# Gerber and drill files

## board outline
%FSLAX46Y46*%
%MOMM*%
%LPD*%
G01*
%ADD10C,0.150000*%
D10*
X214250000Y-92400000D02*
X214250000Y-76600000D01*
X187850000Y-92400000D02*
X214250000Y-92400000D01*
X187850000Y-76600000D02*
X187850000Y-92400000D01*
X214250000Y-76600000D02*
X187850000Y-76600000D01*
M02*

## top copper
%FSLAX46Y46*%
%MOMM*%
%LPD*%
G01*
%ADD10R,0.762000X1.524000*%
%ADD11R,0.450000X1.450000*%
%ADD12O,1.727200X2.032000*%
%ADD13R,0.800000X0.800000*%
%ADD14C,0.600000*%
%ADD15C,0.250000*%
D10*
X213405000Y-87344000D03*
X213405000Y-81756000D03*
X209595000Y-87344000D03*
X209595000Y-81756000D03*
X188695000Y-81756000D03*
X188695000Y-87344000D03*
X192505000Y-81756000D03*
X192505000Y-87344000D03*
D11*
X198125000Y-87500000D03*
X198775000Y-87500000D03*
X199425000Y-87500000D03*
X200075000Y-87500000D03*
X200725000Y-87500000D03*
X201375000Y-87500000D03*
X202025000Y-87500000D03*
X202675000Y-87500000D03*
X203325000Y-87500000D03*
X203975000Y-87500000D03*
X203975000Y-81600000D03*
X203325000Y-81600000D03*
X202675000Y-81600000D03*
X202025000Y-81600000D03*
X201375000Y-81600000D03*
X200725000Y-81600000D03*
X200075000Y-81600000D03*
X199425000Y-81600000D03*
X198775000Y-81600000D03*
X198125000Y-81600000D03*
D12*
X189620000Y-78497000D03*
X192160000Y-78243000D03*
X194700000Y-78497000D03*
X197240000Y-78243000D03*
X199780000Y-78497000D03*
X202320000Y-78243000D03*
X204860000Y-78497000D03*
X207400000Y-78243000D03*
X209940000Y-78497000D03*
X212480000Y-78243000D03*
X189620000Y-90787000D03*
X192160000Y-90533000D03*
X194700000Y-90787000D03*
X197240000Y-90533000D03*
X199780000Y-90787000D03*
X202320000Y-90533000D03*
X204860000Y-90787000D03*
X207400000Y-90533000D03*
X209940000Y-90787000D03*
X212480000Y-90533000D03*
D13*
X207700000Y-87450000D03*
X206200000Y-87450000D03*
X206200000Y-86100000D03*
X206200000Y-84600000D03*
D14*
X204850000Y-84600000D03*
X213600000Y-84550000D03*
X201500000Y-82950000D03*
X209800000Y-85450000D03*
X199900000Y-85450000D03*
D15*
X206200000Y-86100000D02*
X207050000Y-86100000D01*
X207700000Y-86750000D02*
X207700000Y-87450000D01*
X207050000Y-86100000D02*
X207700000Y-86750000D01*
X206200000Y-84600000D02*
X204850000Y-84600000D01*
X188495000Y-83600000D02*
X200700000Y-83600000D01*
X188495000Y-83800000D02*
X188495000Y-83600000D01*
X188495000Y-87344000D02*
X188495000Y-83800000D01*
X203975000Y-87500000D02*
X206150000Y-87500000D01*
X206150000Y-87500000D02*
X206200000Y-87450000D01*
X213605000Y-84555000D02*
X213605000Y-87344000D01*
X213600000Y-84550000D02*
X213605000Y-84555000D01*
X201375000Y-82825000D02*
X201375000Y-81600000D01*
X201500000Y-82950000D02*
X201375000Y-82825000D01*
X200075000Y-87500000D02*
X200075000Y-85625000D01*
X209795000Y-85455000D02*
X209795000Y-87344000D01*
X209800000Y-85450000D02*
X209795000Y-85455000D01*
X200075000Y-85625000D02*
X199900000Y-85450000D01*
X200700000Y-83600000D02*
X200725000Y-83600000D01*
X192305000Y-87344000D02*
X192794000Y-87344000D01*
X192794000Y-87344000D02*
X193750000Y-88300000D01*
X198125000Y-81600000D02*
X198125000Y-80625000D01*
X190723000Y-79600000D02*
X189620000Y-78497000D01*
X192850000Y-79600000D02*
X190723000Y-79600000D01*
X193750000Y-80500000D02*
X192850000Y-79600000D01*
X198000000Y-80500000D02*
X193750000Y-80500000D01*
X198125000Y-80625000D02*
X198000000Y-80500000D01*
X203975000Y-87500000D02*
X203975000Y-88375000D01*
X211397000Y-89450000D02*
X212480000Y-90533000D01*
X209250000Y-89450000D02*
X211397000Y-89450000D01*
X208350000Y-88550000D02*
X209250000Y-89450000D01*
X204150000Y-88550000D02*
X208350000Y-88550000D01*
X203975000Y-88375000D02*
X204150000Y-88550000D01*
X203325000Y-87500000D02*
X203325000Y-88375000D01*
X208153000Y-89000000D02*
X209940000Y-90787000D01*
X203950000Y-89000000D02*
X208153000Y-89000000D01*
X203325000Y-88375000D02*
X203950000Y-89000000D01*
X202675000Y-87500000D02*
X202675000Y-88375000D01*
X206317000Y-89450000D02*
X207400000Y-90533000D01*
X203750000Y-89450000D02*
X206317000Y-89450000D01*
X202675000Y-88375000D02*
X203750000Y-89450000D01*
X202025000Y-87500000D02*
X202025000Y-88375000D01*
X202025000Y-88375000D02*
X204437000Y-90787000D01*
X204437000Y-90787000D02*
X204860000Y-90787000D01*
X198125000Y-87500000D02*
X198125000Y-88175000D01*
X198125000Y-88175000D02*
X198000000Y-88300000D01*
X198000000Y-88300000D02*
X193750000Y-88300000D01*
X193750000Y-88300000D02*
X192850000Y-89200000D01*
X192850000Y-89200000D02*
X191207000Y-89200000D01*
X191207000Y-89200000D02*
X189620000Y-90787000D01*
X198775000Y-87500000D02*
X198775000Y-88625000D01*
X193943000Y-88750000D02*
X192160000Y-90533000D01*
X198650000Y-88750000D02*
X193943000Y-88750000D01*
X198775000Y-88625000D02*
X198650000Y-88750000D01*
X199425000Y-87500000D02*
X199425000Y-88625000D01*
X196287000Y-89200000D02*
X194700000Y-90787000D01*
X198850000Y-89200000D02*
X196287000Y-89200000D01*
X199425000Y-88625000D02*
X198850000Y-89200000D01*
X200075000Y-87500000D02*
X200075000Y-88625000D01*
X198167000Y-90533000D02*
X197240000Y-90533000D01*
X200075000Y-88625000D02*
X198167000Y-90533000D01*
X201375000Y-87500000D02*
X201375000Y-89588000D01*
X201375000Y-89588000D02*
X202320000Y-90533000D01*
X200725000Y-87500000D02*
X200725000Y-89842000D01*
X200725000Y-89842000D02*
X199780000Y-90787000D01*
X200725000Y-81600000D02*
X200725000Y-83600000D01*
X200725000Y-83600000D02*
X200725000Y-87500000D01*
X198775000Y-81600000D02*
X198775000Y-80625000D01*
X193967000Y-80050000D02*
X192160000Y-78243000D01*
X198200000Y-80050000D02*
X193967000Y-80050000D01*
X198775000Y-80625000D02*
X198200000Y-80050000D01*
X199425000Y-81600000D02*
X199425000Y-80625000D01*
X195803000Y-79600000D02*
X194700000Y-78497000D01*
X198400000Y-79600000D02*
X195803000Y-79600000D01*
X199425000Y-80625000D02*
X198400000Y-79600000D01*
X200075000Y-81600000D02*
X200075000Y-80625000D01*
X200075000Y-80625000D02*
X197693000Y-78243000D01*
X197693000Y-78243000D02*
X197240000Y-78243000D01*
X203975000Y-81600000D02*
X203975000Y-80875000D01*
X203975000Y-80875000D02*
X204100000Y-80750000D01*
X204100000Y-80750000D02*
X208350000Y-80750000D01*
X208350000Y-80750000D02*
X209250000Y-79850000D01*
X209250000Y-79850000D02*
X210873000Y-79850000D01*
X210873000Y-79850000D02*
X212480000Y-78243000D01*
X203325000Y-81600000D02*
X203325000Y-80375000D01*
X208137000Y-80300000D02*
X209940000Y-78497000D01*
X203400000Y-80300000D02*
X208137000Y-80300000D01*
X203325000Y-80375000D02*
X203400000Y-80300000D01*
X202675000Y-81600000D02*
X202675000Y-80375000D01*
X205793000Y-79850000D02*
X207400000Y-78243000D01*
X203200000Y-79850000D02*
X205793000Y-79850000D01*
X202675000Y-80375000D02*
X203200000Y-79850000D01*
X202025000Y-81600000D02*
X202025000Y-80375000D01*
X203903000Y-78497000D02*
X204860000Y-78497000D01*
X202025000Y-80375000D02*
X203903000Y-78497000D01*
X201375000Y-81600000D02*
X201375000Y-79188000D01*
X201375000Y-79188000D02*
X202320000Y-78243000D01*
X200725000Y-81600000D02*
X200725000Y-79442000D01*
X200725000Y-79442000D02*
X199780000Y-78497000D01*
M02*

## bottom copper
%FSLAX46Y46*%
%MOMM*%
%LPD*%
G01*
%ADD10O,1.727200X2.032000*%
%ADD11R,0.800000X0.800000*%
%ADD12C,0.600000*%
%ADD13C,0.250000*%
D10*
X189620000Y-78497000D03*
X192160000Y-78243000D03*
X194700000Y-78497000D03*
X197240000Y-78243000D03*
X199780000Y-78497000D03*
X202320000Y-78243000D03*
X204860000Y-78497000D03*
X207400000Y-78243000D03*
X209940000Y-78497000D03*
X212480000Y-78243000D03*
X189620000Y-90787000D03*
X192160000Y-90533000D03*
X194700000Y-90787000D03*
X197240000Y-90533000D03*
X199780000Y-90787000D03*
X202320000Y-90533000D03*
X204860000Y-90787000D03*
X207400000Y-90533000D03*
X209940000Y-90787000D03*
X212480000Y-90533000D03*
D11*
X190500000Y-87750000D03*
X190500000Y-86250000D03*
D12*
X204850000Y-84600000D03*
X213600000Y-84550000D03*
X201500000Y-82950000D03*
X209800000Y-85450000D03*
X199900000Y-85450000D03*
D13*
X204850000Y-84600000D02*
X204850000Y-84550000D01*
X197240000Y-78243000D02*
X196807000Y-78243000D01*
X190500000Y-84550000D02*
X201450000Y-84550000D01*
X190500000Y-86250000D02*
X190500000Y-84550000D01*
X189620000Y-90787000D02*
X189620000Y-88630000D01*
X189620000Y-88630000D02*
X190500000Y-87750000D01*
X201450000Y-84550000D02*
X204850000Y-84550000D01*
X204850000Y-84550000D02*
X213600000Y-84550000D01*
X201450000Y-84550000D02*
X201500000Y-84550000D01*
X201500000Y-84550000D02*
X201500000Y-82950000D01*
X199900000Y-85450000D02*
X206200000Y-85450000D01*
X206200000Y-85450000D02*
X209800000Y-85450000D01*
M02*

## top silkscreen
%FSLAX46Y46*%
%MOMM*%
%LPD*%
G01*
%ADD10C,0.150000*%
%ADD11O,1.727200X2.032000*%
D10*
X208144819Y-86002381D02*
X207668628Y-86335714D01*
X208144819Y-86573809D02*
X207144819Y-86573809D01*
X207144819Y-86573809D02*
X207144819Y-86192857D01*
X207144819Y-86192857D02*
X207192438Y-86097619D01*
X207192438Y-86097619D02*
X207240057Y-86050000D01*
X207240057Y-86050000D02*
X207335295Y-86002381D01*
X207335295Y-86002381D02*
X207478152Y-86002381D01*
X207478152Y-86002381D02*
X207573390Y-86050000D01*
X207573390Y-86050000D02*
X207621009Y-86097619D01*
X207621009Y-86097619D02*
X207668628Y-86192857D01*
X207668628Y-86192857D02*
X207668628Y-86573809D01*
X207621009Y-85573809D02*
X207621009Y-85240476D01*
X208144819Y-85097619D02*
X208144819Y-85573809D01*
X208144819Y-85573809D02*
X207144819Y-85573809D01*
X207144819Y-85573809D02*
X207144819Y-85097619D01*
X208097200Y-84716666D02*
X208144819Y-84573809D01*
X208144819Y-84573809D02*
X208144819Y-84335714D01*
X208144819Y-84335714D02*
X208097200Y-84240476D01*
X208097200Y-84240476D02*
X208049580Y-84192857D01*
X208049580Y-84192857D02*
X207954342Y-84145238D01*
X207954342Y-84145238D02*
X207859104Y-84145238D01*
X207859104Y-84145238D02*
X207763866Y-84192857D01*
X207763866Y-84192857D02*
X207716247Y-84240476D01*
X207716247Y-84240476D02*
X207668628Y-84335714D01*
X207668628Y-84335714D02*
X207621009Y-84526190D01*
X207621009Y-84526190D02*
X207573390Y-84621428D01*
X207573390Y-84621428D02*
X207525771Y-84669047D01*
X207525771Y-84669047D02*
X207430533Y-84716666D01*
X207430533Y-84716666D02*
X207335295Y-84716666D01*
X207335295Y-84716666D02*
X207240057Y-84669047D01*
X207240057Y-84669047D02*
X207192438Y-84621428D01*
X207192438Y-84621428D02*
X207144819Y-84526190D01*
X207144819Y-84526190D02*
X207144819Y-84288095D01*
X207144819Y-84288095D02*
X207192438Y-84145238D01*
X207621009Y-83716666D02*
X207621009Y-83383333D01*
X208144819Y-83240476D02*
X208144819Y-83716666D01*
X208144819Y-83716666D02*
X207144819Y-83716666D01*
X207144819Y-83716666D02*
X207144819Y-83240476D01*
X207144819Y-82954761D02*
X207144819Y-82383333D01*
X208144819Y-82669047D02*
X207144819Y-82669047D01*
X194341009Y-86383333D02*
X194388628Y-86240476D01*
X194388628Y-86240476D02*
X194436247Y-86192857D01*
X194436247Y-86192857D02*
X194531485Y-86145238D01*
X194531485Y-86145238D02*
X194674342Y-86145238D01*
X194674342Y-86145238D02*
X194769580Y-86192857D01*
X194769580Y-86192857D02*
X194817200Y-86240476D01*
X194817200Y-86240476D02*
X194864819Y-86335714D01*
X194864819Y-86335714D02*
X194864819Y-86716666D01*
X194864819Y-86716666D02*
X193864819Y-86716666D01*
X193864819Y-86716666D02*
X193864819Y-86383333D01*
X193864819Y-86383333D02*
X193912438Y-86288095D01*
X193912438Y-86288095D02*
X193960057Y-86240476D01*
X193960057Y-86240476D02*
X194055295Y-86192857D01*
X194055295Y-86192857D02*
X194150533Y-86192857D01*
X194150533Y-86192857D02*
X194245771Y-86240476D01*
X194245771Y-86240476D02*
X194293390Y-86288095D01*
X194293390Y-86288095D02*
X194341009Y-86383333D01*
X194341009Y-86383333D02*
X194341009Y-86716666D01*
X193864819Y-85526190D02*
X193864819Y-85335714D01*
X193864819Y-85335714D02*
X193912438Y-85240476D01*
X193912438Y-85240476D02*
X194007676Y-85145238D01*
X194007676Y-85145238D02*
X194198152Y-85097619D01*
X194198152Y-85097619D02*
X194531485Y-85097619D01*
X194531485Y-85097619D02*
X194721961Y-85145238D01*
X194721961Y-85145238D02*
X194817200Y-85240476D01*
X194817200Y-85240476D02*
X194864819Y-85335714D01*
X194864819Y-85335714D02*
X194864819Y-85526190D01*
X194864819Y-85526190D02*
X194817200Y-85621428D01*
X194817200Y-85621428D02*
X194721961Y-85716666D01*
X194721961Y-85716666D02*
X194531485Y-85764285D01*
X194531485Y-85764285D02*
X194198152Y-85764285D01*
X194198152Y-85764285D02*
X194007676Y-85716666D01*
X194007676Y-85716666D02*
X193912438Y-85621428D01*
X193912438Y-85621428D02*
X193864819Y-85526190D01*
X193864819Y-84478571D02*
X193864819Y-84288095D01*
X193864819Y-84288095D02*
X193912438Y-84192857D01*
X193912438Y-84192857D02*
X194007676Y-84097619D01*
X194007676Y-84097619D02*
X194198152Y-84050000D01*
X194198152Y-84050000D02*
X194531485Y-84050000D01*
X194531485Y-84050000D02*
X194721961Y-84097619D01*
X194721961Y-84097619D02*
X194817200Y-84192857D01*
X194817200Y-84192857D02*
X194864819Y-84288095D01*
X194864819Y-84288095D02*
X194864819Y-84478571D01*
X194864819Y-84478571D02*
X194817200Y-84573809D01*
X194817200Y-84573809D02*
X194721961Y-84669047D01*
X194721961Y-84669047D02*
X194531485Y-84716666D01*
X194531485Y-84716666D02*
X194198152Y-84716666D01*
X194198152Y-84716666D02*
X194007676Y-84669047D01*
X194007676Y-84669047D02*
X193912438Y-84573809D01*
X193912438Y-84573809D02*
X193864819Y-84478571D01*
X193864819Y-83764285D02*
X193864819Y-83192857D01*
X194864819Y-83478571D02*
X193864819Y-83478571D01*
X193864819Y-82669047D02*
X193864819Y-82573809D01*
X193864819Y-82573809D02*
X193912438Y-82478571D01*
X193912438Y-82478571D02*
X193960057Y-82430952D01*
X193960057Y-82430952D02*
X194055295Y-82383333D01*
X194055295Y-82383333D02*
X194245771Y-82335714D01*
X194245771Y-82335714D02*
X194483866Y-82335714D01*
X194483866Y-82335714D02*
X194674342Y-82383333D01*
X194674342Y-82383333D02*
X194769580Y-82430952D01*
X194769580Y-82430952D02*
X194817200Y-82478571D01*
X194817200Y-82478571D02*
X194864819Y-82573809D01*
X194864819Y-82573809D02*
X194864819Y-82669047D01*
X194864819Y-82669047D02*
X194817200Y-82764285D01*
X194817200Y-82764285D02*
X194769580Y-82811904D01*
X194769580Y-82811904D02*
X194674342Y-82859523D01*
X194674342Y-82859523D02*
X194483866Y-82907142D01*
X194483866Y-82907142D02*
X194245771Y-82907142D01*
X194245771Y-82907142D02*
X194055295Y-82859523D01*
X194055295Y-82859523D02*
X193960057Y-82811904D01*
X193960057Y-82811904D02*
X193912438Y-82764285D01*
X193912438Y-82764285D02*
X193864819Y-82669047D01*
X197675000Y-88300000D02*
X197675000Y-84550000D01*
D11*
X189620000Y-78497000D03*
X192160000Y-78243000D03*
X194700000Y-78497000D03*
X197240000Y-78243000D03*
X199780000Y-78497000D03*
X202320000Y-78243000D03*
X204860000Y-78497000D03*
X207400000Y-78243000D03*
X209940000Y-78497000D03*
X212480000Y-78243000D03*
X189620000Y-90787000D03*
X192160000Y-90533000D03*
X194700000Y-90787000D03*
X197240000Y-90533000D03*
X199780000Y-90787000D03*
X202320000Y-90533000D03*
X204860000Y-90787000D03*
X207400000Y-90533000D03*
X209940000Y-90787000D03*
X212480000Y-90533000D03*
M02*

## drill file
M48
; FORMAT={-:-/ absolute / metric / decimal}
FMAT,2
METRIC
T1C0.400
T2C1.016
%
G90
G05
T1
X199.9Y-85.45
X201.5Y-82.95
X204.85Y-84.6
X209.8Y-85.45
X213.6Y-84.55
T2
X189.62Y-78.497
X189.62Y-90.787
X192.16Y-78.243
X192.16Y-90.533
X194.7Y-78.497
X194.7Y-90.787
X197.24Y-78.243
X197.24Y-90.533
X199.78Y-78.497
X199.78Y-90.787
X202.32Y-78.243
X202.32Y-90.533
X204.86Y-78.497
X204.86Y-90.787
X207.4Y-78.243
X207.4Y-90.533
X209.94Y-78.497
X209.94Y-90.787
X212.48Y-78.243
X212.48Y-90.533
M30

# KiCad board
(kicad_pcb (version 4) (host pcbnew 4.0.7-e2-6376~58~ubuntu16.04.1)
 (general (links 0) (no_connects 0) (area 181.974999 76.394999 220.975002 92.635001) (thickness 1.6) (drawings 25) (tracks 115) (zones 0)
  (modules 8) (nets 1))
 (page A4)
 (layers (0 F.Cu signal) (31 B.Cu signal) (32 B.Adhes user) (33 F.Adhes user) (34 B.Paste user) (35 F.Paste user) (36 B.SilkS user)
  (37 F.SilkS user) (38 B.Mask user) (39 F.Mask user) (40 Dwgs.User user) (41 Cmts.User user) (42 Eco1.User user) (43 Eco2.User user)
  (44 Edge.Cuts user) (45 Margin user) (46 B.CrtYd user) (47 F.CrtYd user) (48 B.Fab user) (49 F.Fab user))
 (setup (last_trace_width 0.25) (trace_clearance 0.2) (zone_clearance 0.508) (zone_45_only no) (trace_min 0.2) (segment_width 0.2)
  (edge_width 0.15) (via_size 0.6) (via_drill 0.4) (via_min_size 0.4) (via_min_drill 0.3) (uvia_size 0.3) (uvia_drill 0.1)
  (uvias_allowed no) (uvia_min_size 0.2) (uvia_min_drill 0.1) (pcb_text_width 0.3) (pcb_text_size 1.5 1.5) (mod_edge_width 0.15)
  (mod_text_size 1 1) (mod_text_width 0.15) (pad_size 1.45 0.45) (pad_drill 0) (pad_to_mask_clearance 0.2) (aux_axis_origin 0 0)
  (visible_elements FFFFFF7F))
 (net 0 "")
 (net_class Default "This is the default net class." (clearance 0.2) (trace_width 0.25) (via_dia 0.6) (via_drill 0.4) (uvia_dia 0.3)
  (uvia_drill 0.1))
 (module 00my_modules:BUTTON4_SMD (layer F.Cu) (at 211.5 84.55 90)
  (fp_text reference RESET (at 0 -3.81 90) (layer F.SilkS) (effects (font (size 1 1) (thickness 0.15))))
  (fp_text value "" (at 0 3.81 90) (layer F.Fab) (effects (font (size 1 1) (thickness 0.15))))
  (pad 1 smd rect (at -2.794 1.905 90) (size 1.524 0.762) (layers F.Cu F.Paste F.Mask))
  (pad 2 smd rect (at 2.794 1.905 90) (size 1.524 0.762) (layers F.Cu F.Paste F.Mask))
  (pad 3 smd rect (at -2.794 -1.905 90) (size 1.524 0.762) (layers F.Cu F.Paste F.Mask))
  (pad 4 smd rect (at 2.794 -1.905 90) (size 1.524 0.762) (layers F.Cu F.Paste F.Mask)))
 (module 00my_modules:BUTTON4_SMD (layer F.Cu) (at 190.6 84.55 270)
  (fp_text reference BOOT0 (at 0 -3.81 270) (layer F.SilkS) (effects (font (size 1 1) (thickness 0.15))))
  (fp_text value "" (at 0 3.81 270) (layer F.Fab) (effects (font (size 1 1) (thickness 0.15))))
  (pad 1 smd rect (at -2.794 1.905 270) (size 1.524 0.762) (layers F.Cu F.Paste F.Mask))
  (pad 2 smd rect (at 2.794 1.905 270) (size 1.524 0.762) (layers F.Cu F.Paste F.Mask))
  (pad 3 smd rect (at -2.794 -1.905 270) (size 1.524 0.762) (layers F.Cu F.Paste F.Mask))
  (pad 4 smd rect (at 2.794 -1.905 270) (size 1.524 0.762) (layers F.Cu F.Paste F.Mask)))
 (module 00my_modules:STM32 (layer F.Cu) (at 201.05 84.55 90)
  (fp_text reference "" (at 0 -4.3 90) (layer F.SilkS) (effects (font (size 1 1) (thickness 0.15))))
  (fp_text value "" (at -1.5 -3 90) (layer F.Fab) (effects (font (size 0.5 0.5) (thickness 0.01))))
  (fp_line (start -3.75 -3.375) (end 0 -3.375) (layer F.SilkS) (width 0.15))
  (pad BOOT smd rect (at -2.95 -2.925 90) (size 1.45 0.45) (layers F.Cu F.Paste F.Mask))
  (pad PF0 smd rect (at -2.95 -2.275 90) (size 1.45 0.45) (layers F.Cu F.Paste F.Mask))
  (pad PF1 smd rect (at -2.95 -1.625 90) (size 1.45 0.45) (layers F.Cu F.Paste F.Mask))
  (pad NRST smd rect (at -2.95 -0.975 90) (size 1.45 0.45) (layers F.Cu F.Paste F.Mask))
  (pad VCC smd rect (at -2.95 -0.325 90) (size 1.45 0.45) (layers F.Cu F.Paste F.Mask))
  (pad PA0 smd rect (at -2.95 0.325 90) (size 1.45 0.45) (layers F.Cu F.Paste F.Mask))
  (pad PA1 smd rect (at -2.95 0.975 90) (size 1.45 0.45) (layers F.Cu F.Paste F.Mask))
  (pad PA2 smd rect (at -2.95 1.625 90) (size 1.45 0.45) (layers F.Cu F.Paste F.Mask))
  (pad PA3 smd rect (at -2.95 2.275 90) (size 1.45 0.45) (layers F.Cu F.Paste F.Mask))
  (pad PA4 smd rect (at -2.95 2.925 90) (size 1.45 0.45) (layers F.Cu F.Paste F.Mask))
  (pad PA5 smd rect (at 2.95 2.925 90) (size 1.45 0.45) (layers F.Cu F.Paste F.Mask))
  (pad PA6 smd rect (at 2.95 2.275 90) (size 1.45 0.45) (layers F.Cu F.Paste F.Mask))
  (pad PA7 smd rect (at 2.95 1.625 90) (size 1.45 0.45) (layers F.Cu F.Paste F.Mask))
  (pad PB1 smd rect (at 2.95 0.975 90) (size 1.45 0.45) (layers F.Cu F.Paste F.Mask))
  (pad GND smd rect (at 2.95 0.325 90) (size 1.45 0.45) (layers F.Cu F.Paste F.Mask))
  (pad VCC smd rect (at 2.95 -0.325 90) (size 1.45 0.45) (layers F.Cu F.Paste F.Mask))
  (pad TX smd rect (at 2.95 -0.975 90) (size 1.45 0.45) (layers F.Cu F.Paste F.Mask))
  (pad RX smd rect (at 2.95 -1.625 90) (size 1.45 0.45) (layers F.Cu F.Paste F.Mask))
  (pad DIO smd rect (at 2.95 -2.275 90) (size 1.45 0.45) (layers F.Cu F.Paste F.Mask))
  (pad CLK smd rect (at 2.95 -2.925 90) (size 1.45 0.45) (layers F.Cu F.Paste F.Mask)))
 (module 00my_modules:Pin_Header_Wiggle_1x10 (layer F.Cu) (at 189.62 78.37 90)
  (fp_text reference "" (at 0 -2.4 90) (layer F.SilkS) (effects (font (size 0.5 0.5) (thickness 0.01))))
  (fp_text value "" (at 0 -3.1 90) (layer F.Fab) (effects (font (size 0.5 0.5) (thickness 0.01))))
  (pad 1 thru_hole oval (at -0.127 0 90) (size 2.032 1.7272) (drill 1.016) (layers *.Cu *.Mask F.SilkS))
  (pad 2 thru_hole oval (at 0.127 2.54 90) (size 2.032 1.7272) (drill 1.016) (layers *.Cu *.Mask F.SilkS))
  (pad 3 thru_hole oval (at -0.127 5.08 90) (size 2.032 1.7272) (drill 1.016) (layers *.Cu *.Mask F.SilkS))
  (pad 4 thru_hole oval (at 0.127 7.62 90) (size 2.032 1.7272) (drill 1.016) (layers *.Cu *.Mask F.SilkS))
  (pad 5 thru_hole oval (at -0.127 10.16 90) (size 2.032 1.7272) (drill 1.016) (layers *.Cu *.Mask F.SilkS))
  (pad 6 thru_hole oval (at 0.127 12.7 90) (size 2.032 1.7272) (drill 1.016) (layers *.Cu *.Mask F.SilkS))
  (pad 7 thru_hole oval (at -0.127 15.24 90) (size 2.032 1.7272) (drill 1.016) (layers *.Cu *.Mask F.SilkS))
  (pad 8 thru_hole oval (at 0.127 17.78 90) (size 2.032 1.7272) (drill 1.016) (layers *.Cu *.Mask F.SilkS))
  (pad 9 thru_hole oval (at -0.127 20.32 90) (size 2.032 1.7272) (drill 1.016) (layers *.Cu *.Mask F.SilkS))
  (pad 10 thru_hole oval (at 0.127 22.86 90) (size 2.032 1.7272) (drill 1.016) (layers *.Cu *.Mask F.SilkS)))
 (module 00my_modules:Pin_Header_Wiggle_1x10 (layer F.Cu) (at 189.62 90.66 90)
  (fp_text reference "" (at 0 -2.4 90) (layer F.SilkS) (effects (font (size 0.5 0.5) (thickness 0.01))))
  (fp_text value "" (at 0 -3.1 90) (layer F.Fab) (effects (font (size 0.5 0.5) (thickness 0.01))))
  (pad 1 thru_hole oval (at -0.127 0 90) (size 2.032 1.7272) (drill 1.016) (layers *.Cu *.Mask F.SilkS))
  (pad 2 thru_hole oval (at 0.127 2.54 90) (size 2.032 1.7272) (drill 1.016) (layers *.Cu *.Mask F.SilkS))
  (pad 3 thru_hole oval (at -0.127 5.08 90) (size 2.032 1.7272) (drill 1.016) (layers *.Cu *.Mask F.SilkS))
  (pad 4 thru_hole oval (at 0.127 7.62 90) (size 2.032 1.7272) (drill 1.016) (layers *.Cu *.Mask F.SilkS))
  (pad 5 thru_hole oval (at -0.127 10.16 90) (size 2.032 1.7272) (drill 1.016) (layers *.Cu *.Mask F.SilkS))
  (pad 6 thru_hole oval (at 0.127 12.7 90) (size 2.032 1.7272) (drill 1.016) (layers *.Cu *.Mask F.SilkS))
  (pad 7 thru_hole oval (at -0.127 15.24 90) (size 2.032 1.7272) (drill 1.016) (layers *.Cu *.Mask F.SilkS))
  (pad 8 thru_hole oval (at 0.127 17.78 90) (size 2.032 1.7272) (drill 1.016) (layers *.Cu *.Mask F.SilkS))
  (pad 9 thru_hole oval (at -0.127 20.32 90) (size 2.032 1.7272) (drill 1.016) (layers *.Cu *.Mask F.SilkS))
  (pad 10 thru_hole oval (at 0.127 22.86 90) (size 2.032 1.7272) (drill 1.016) (layers *.Cu *.Mask F.SilkS)))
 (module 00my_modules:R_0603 (layer B.Cu) (at 190.5 87 90)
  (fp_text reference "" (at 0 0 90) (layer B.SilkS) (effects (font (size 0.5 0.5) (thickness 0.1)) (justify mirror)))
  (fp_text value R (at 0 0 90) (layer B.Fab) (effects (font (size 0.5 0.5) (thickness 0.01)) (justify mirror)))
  (pad 1 smd rect (at -0.75 0 90) (size 0.8 0.8) (layers B.Cu B.Paste B.Mask))
  (pad 2 smd rect (at 0.75 0 90) (size 0.8 0.8) (layers B.Cu B.Paste B.Mask)))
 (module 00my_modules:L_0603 (layer F.Cu) (at 206.95 87.45 180)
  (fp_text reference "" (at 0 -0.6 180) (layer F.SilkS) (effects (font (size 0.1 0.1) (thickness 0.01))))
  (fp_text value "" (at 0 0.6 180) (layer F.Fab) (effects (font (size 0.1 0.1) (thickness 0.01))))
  (pad 1 smd rect (at -0.75 0 180) (size 0.8 0.8) (layers F.Cu F.Paste F.Mask))
  (pad 2 smd rect (at 0.75 0 180) (size 0.8 0.8) (layers F.Cu F.Paste F.Mask)))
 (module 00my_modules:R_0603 (layer F.Cu) (at 206.2 85.35 90)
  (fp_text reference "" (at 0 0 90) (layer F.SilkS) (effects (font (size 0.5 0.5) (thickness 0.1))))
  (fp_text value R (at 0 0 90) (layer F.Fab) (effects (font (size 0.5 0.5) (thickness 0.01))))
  (pad 1 smd rect (at -0.75 0 90) (size 0.8 0.8) (layers F.Cu F.Paste F.Mask))
  (pad 2 smd rect (at 0.75 0 90) (size 0.8 0.8) (layers F.Cu F.Paste F.Mask)))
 (gr_line (start 214.25 92.4) (end 214.25 76.6) (angle 90) (layer Edge.Cuts) (width 0.15))
 (gr_line (start 187.85 92.4) (end 214.25 92.4) (angle 90) (layer Edge.Cuts) (width 0.15))
 (gr_line (start 187.85 76.6) (end 187.85 92.4) (angle 90) (layer Edge.Cuts) (width 0.15))
 (gr_line (start 214.25 76.6) (end 187.85 76.6) (angle 90) (layer Edge.Cuts) (width 0.15))
 (segment (start 206.2 86.1) (end 207.05 86.1) (width 0.25) (layer F.Cu) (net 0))
 (segment (start 207.7 86.75) (end 207.7 87.45) (width 0.25) (layer F.Cu) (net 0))
 (segment (start 207.05 86.1) (end 207.7 86.75) (width 0.25) (layer F.Cu) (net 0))
 (segment (start 206.2 84.6) (end 204.85 84.6) (width 0.25) (layer F.Cu) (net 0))
 (segment (start 204.85 84.6) (end 204.85 84.55) (width 0.25) (layer B.Cu) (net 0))
 (via (at 204.85 84.6) (size 0.6) (drill 0.4) (layers F.Cu B.Cu) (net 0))
 (segment (start 188.495 83.6) (end 200.7 83.6) (width 0.25) (layer F.Cu) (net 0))
 (segment (start 188.495 83.8) (end 188.495 83.6) (width 0.25) (layer F.Cu) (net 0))
 (segment (start 188.495 87.344) (end 188.495 83.8) (width 0.25) (layer F.Cu) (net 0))
 (segment (start 203.975 87.5) (end 206.15 87.5) (width 0.25) (layer F.Cu) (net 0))
 (segment (start 206.15 87.5) (end 206.2 87.45) (width 0.25) (layer F.Cu) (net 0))
 (segment (start 197.24 78.243) (end 196.807 78.243) (width 0.25) (layer B.Cu) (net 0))
 (segment (start 190.5 84.55) (end 201.45 84.55) (width 0.25) (layer B.Cu) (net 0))
 (segment (start 190.5 86.25) (end 190.5 84.55) (width 0.25) (layer B.Cu) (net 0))
 (segment (start 189.62 90.787) (end 189.62 88.63) (width 0.25) (layer B.Cu) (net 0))
 (segment (start 189.62 88.63) (end 190.5 87.75) (width 0.25) (layer B.Cu) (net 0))
 (segment (start 201.45 84.55) (end 204.85 84.55) (width 0.25) (layer B.Cu) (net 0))
 (segment (start 204.85 84.55) (end 213.6 84.55) (width 0.25) (layer B.Cu) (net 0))
 (via (at 213.6 84.55) (size 0.6) (drill 0.4) (layers F.Cu B.Cu) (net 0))
 (segment (start 213.605 84.555) (end 213.605 87.344) (width 0.25) (layer F.Cu) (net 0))
 (segment (start 213.6 84.55) (end 213.605 84.555) (width 0.25) (layer F.Cu) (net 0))
 (segment (start 201.45 84.55) (end 201.5 84.55) (width 0.25) (layer B.Cu) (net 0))
 (segment (start 201.375 82.825) (end 201.375 81.6) (width 0.25) (layer F.Cu) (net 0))
 (segment (start 201.5 82.95) (end 201.375 82.825) (width 0.25) (layer F.Cu) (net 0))
 (via (at 201.5 82.95) (size 0.6) (drill 0.4) (layers F.Cu B.Cu) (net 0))
 (segment (start 201.5 84.55) (end 201.5 82.95) (width 0.25) (layer B.Cu) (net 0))
 (segment (start 200.075 87.5) (end 200.075 85.625) (width 0.25) (layer F.Cu) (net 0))
 (segment (start 209.795 85.455) (end 209.795 87.344) (width 0.25) (layer F.Cu) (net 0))
 (segment (start 209.8 85.45) (end 209.795 85.455) (width 0.25) (layer F.Cu) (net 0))
 (via (at 209.8 85.45) (size 0.6) (drill 0.4) (layers F.Cu B.Cu) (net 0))
 (segment (start 199.9 85.45) (end 206.2 85.45) (width 0.25) (layer B.Cu) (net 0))
 (segment (start 206.2 85.45) (end 209.8 85.45) (width 0.25) (layer B.Cu) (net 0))
 (via (at 199.9 85.45) (size 0.6) (drill 0.4) (layers F.Cu B.Cu) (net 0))
 (segment (start 200.075 85.625) (end 199.9 85.45) (width 0.25) (layer F.Cu) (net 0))
 (segment (start 200.7 83.6) (end 200.725 83.6) (width 0.25) (layer F.Cu) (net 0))
 (segment (start 192.305 87.344) (end 192.794 87.344) (width 0.25) (layer F.Cu) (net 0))
 (segment (start 192.794 87.344) (end 193.75 88.3) (width 0.25) (layer F.Cu) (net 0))
 (segment (start 198.125 81.6) (end 198.125 80.625) (width 0.25) (layer F.Cu) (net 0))
 (segment (start 190.723 79.6) (end 189.62 78.497) (width 0.25) (layer F.Cu) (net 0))
 (segment (start 192.85 79.6) (end 190.723 79.6) (width 0.25) (layer F.Cu) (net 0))
 (segment (start 193.75 80.5) (end 192.85 79.6) (width 0.25) (layer F.Cu) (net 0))
 (segment (start 198 80.5) (end 193.75 80.5) (width 0.25) (layer F.Cu) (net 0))
 (segment (start 198.125 80.625) (end 198 80.5) (width 0.25) (layer F.Cu) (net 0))
 (segment (start 203.975 87.5) (end 203.975 88.375) (width 0.25) (layer F.Cu) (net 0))
 (segment (start 211.397 89.45) (end 212.48 90.533) (width 0.25) (layer F.Cu) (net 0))
 (segment (start 209.25 89.45) (end 211.397 89.45) (width 0.25) (layer F.Cu) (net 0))
 (segment (start 208.35 88.55) (end 209.25 89.45) (width 0.25) (layer F.Cu) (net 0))
 (segment (start 204.15 88.55) (end 208.35 88.55) (width 0.25) (layer F.Cu) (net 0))
 (segment (start 203.975 88.375) (end 204.15 88.55) (width 0.25) (layer F.Cu) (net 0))
 (segment (start 203.325 87.5) (end 203.325 88.375) (width 0.25) (layer F.Cu) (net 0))
 (segment (start 208.153 89) (end 209.94 90.787) (width 0.25) (layer F.Cu) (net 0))
 (segment (start 203.95 89) (end 208.153 89) (width 0.25) (layer F.Cu) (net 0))
 (segment (start 203.325 88.375) (end 203.95 89) (width 0.25) (layer F.Cu) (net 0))
 (segment (start 202.675 87.5) (end 202.675 88.375) (width 0.25) (layer F.Cu) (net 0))
 (segment (start 206.317 89.45) (end 207.4 90.533) (width 0.25) (layer F.Cu) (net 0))
 (segment (start 203.75 89.45) (end 206.317 89.45) (width 0.25) (layer F.Cu) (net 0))
 (segment (start 202.675 88.375) (end 203.75 89.45) (width 0.25) (layer F.Cu) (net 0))
 (segment (start 202.025 87.5) (end 202.025 88.375) (width 0.25) (layer F.Cu) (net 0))
 (segment (start 202.025 88.375) (end 204.437 90.787) (width 0.25) (layer F.Cu) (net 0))
 (segment (start 204.437 90.787) (end 204.86 90.787) (width 0.25) (layer F.Cu) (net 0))
 (segment (start 198.125 87.5) (end 198.125 88.175) (width 0.25) (layer F.Cu) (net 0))
 (segment (start 198.125 88.175) (end 198 88.3) (width 0.25) (layer F.Cu) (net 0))
 (segment (start 198 88.3) (end 193.75 88.3) (width 0.25) (layer F.Cu) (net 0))
 (segment (start 193.75 88.3) (end 192.85 89.2) (width 0.25) (layer F.Cu) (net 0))
 (segment (start 192.85 89.2) (end 191.207 89.2) (width 0.25) (layer F.Cu) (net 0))
 (segment (start 191.207 89.2) (end 189.62 90.787) (width 0.25) (layer F.Cu) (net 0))
 (segment (start 198.775 87.5) (end 198.775 88.625) (width 0.25) (layer F.Cu) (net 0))
 (segment (start 193.943 88.75) (end 192.16 90.533) (width 0.25) (layer F.Cu) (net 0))
 (segment (start 198.65 88.75) (end 193.943 88.75) (width 0.25) (layer F.Cu) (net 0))
 (segment (start 198.775 88.625) (end 198.65 88.75) (width 0.25) (layer F.Cu) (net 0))
 (segment (start 199.425 87.5) (end 199.425 88.625) (width 0.25) (layer F.Cu) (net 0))
 (segment (start 196.287 89.2) (end 194.7 90.787) (width 0.25) (layer F.Cu) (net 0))
 (segment (start 198.85 89.2) (end 196.287 89.2) (width 0.25) (layer F.Cu) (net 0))
 (segment (start 199.425 88.625) (end 198.85 89.2) (width 0.25) (layer F.Cu) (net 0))
 (segment (start 200.075 87.5) (end 200.075 88.625) (width 0.25) (layer F.Cu) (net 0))
 (segment (start 198.167 90.533) (end 197.24 90.533) (width 0.25) (layer F.Cu) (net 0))
 (segment (start 200.075 88.625) (end 198.167 90.533) (width 0.25) (layer F.Cu) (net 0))
 (segment (start 201.375 87.5) (end 201.375 89.588) (width 0.25) (layer F.Cu) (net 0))
 (segment (start 201.375 89.588) (end 202.32 90.533) (width 0.25) (layer F.Cu) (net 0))
 (segment (start 200.725 87.5) (end 200.725 89.842) (width 0.25) (layer F.Cu) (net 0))
 (segment (start 200.725 89.842) (end 199.78 90.787) (width 0.25) (layer F.Cu) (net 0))
 (segment (start 200.725 81.6) (end 200.725 83.6) (width 0.25) (layer F.Cu) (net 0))
 (segment (start 200.725 83.6) (end 200.725 87.5) (width 0.25) (layer F.Cu) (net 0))
 (segment (start 198.775 81.6) (end 198.775 80.625) (width 0.25) (layer F.Cu) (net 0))
 (segment (start 193.967 80.05) (end 192.16 78.243) (width 0.25) (layer F.Cu) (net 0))
 (segment (start 198.2 80.05) (end 193.967 80.05) (width 0.25) (layer F.Cu) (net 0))
 (segment (start 198.775 80.625) (end 198.2 80.05) (width 0.25) (layer F.Cu) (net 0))
 (segment (start 199.425 81.6) (end 199.425 80.625) (width 0.25) (layer F.Cu) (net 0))
 (segment (start 195.803 79.6) (end 194.7 78.497) (width 0.25) (layer F.Cu) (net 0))
 (segment (start 198.4 79.6) (end 195.803 79.6) (width 0.25) (layer F.Cu) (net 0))
 (segment (start 199.425 80.625) (end 198.4 79.6) (width 0.25) (layer F.Cu) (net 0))
 (segment (start 200.075 81.6) (end 200.075 80.625) (width 0.25) (layer F.Cu) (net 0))
 (segment (start 200.075 80.625) (end 197.693 78.243) (width 0.25) (layer F.Cu) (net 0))
 (segment (start 197.693 78.243) (end 197.24 78.243) (width 0.25) (layer F.Cu) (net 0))
 (segment (start 203.975 81.6) (end 203.975 80.875) (width 0.25) (layer F.Cu) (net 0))
 (segment (start 203.975 80.875) (end 204.1 80.75) (width 0.25) (layer F.Cu) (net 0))
 (segment (start 204.1 80.75) (end 208.35 80.75) (width 0.25) (layer F.Cu) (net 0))
 (segment (start 208.35 80.75) (end 209.25 79.85) (width 0.25) (layer F.Cu) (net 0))
 (segment (start 209.25 79.85) (end 210.873 79.85) (width 0.25) (layer F.Cu) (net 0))
 (segment (start 210.873 79.85) (end 212.48 78.243) (width 0.25) (layer F.Cu) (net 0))
 (segment (start 203.325 81.6) (end 203.325 80.375) (width 0.25) (layer F.Cu) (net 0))
 (segment (start 208.137 80.3) (end 209.94 78.497) (width 0.25) (layer F.Cu) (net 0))
 (segment (start 203.4 80.3) (end 208.137 80.3) (width 0.25) (layer F.Cu) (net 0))
 (segment (start 203.325 80.375) (end 203.4 80.3) (width 0.25) (layer F.Cu) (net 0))
 (segment (start 202.675 81.6) (end 202.675 80.375) (width 0.25) (layer F.Cu) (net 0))
 (segment (start 205.793 79.85) (end 207.4 78.243) (width 0.25) (layer F.Cu) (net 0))
 (segment (start 203.2 79.85) (end 205.793 79.85) (width 0.25) (layer F.Cu) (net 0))
 (segment (start 202.675 80.375) (end 203.2 79.85) (width 0.25) (layer F.Cu) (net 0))
 (segment (start 202.025 81.6) (end 202.025 80.375) (width 0.25) (layer F.Cu) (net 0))
 (segment (start 203.903 78.497) (end 204.86 78.497) (width 0.25) (layer F.Cu) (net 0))
 (segment (start 202.025 80.375) (end 203.903 78.497) (width 0.25) (layer F.Cu) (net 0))
 (segment (start 201.375 81.6) (end 201.375 79.188) (width 0.25) (layer F.Cu) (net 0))
 (segment (start 201.375 79.188) (end 202.32 78.243) (width 0.25) (layer F.Cu) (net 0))
 (segment (start 200.725 81.6) (end 200.725 79.442) (width 0.25) (layer F.Cu) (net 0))
 (segment (start 200.725 79.442) (end 199.78 78.497) (width 0.25) (layer F.Cu) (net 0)))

